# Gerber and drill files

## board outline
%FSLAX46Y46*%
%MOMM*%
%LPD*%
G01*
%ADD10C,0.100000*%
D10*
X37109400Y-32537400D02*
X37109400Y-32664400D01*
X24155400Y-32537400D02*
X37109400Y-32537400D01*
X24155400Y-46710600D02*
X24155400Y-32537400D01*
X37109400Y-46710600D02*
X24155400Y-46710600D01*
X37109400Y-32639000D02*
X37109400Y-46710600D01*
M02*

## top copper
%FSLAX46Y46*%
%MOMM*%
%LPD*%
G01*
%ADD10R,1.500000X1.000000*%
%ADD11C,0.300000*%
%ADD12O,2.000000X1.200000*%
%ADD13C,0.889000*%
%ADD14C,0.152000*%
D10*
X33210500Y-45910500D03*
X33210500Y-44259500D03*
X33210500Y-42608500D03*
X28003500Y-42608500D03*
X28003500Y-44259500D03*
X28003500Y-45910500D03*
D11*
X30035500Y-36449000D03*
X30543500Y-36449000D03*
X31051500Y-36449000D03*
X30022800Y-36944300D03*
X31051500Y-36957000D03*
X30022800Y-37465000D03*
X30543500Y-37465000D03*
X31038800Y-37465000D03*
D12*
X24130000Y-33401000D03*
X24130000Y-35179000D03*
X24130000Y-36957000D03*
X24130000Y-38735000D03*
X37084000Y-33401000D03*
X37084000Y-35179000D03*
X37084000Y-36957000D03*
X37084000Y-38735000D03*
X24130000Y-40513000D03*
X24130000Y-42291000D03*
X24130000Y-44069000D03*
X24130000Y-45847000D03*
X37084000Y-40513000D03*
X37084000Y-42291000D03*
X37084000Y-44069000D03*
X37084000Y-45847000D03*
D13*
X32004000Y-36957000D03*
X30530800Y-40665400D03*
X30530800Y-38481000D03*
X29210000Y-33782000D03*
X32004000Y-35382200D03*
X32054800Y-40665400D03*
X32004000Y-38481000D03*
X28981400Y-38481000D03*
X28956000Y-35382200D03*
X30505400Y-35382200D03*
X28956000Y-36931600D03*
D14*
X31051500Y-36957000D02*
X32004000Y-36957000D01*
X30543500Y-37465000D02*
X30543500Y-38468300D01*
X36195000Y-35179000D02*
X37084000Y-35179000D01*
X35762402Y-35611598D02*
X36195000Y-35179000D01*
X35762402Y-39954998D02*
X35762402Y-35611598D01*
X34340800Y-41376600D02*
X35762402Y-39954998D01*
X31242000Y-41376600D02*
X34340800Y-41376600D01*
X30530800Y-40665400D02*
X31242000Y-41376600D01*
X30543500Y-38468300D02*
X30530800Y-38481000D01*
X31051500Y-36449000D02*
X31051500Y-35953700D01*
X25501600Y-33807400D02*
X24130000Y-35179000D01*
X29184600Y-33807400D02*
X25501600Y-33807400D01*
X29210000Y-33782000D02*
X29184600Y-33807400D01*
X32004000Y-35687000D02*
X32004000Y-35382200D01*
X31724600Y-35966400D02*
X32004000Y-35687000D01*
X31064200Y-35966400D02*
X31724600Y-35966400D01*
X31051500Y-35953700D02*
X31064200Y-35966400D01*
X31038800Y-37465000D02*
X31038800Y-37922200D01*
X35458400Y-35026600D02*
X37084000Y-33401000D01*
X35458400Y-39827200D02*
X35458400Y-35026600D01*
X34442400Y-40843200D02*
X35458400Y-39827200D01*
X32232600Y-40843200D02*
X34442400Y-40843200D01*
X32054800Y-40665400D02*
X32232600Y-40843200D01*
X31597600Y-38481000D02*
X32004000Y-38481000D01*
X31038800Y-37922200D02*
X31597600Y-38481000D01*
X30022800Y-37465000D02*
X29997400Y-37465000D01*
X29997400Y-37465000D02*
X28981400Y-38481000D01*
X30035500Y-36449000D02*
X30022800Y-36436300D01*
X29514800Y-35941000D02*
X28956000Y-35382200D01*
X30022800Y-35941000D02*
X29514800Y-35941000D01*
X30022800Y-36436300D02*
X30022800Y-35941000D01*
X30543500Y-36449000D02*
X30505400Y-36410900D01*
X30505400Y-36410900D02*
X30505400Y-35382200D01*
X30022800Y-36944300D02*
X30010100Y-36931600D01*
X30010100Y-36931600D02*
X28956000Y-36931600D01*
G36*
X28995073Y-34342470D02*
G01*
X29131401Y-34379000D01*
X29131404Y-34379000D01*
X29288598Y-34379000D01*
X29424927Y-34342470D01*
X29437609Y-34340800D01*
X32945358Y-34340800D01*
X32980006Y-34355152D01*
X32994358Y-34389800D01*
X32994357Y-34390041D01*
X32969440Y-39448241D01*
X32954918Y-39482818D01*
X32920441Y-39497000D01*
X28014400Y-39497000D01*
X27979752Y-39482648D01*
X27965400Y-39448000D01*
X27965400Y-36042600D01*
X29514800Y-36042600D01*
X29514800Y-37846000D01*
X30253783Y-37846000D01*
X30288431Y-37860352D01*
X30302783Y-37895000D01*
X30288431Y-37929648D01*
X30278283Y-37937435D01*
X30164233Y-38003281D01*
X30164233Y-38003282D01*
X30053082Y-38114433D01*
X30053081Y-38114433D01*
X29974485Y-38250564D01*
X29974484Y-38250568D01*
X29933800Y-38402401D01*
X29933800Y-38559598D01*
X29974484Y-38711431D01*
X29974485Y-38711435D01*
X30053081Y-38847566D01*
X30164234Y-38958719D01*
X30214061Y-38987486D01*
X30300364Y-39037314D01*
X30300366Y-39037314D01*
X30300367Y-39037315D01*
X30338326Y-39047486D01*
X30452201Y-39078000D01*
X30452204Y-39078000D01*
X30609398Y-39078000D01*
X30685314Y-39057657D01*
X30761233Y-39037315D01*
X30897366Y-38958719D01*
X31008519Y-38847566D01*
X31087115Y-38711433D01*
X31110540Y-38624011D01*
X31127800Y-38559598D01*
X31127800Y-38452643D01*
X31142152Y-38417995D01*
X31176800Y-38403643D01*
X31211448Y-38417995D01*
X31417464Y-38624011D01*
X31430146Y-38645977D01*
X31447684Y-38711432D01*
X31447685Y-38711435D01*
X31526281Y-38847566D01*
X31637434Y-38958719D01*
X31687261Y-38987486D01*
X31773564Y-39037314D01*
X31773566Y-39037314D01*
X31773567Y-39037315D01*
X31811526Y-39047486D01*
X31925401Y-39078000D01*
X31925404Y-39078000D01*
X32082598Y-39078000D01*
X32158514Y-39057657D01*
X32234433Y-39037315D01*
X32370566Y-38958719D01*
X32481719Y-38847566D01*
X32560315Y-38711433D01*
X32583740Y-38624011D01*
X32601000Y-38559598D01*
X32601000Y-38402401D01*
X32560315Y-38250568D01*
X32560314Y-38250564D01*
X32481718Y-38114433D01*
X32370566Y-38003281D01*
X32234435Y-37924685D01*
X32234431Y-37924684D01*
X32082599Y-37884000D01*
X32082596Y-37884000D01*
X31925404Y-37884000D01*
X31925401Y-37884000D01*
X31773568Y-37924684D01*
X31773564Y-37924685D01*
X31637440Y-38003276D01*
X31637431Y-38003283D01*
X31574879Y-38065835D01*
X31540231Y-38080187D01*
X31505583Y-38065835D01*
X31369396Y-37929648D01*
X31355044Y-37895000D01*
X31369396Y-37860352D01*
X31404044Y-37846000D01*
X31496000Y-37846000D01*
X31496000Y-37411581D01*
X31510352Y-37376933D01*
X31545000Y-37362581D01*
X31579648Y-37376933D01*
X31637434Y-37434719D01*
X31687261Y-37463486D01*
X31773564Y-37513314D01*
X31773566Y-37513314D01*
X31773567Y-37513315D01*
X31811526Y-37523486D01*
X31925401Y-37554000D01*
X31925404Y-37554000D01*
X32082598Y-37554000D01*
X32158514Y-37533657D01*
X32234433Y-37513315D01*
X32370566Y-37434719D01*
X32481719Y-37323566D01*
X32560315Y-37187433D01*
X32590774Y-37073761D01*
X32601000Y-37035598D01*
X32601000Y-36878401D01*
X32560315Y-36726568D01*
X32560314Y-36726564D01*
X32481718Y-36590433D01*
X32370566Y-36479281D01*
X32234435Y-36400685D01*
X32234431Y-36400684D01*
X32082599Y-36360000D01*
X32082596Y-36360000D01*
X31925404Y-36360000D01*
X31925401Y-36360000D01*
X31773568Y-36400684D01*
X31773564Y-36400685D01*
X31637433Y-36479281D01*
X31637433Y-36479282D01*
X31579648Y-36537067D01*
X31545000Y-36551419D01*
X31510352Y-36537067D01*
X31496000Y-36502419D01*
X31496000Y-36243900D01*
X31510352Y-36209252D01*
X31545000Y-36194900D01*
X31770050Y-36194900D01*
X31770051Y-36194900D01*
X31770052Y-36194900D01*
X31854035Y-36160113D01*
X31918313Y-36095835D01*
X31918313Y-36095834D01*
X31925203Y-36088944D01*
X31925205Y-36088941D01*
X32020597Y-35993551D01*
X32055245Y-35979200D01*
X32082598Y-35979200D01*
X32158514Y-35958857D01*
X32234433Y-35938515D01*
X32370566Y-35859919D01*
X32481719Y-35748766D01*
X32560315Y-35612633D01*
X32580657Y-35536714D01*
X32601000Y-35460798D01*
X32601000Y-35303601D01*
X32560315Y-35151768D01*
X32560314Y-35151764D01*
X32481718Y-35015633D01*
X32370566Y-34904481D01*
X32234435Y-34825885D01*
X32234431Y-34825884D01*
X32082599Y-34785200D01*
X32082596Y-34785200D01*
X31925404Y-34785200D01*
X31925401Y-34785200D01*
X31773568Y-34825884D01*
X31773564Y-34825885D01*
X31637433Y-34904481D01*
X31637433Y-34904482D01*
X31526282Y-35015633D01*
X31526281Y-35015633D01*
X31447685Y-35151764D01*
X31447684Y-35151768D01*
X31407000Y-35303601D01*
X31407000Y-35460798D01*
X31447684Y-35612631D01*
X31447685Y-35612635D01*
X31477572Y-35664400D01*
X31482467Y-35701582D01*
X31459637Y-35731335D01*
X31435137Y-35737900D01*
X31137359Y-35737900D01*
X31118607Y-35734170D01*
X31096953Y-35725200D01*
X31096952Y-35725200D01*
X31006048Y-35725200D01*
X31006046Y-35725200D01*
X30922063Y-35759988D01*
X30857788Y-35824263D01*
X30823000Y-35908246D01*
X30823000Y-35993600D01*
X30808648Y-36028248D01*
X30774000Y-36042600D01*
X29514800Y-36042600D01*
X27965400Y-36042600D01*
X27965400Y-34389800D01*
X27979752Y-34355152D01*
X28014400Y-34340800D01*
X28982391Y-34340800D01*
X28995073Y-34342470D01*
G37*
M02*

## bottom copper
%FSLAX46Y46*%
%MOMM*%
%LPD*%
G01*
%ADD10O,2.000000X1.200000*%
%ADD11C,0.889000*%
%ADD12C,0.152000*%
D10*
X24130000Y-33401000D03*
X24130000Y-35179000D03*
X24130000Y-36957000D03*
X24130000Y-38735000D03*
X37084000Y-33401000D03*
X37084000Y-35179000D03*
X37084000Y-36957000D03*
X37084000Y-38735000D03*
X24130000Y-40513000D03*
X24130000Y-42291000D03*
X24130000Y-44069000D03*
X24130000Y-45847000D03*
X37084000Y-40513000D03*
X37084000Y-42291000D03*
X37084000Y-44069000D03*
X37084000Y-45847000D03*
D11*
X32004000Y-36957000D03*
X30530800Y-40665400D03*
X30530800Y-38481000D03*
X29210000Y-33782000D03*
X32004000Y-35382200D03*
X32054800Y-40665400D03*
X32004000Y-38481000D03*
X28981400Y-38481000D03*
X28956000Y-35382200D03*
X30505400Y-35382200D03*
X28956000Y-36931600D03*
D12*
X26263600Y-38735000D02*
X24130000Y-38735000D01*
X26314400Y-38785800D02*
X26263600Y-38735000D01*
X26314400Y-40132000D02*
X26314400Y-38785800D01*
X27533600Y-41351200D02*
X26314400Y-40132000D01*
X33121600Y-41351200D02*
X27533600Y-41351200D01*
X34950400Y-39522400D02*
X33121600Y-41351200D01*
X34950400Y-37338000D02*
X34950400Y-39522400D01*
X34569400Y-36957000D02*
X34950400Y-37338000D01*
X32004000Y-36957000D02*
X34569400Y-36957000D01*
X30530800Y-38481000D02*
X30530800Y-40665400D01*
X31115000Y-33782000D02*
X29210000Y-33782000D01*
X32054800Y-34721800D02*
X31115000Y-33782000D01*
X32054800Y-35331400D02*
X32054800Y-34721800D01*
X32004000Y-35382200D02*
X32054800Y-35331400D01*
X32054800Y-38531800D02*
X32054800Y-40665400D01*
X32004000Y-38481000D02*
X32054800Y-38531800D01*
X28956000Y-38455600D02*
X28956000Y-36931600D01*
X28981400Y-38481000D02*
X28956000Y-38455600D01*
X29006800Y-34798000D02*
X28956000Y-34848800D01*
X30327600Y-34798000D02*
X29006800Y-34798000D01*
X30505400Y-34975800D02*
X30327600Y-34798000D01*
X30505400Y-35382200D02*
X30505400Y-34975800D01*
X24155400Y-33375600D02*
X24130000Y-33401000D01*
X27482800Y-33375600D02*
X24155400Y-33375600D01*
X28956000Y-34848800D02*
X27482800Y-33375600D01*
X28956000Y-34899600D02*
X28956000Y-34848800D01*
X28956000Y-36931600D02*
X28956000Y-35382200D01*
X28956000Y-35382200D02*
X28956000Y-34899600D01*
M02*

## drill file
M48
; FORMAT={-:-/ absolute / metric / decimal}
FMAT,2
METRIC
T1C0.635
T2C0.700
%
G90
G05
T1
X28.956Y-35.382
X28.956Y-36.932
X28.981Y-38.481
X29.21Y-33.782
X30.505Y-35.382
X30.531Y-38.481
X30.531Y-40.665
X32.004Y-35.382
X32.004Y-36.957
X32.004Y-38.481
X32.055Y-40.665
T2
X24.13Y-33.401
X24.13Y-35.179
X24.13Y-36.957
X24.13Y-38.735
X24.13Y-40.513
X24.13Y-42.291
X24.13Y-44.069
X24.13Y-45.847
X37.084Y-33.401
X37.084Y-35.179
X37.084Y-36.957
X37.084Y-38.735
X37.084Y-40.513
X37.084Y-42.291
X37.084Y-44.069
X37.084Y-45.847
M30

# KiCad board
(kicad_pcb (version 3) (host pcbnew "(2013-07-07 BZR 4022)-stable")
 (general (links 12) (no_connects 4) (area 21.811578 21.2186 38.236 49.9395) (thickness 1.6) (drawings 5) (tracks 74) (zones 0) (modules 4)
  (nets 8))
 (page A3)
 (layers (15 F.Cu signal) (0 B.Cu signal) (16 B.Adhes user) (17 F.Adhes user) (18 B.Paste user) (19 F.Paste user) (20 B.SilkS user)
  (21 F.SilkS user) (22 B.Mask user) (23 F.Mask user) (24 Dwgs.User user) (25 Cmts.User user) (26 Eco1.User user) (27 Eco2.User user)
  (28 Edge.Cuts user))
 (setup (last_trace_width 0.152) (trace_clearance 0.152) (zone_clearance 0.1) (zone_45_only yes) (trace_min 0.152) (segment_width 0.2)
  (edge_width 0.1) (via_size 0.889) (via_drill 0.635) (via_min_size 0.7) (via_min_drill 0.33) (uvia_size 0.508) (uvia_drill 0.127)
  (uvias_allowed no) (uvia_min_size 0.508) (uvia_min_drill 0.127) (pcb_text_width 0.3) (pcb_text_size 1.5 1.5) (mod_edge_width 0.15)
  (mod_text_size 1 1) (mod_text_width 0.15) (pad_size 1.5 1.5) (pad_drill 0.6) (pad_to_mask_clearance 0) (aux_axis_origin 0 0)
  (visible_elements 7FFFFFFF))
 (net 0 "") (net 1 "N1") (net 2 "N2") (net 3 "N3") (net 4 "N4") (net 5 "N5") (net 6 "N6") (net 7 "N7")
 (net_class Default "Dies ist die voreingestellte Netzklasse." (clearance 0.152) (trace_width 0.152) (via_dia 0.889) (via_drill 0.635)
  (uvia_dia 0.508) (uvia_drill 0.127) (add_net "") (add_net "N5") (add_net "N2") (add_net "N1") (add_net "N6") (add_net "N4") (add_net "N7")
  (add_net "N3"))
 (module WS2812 (layer F.Cu) (at 30.6705 44.2595)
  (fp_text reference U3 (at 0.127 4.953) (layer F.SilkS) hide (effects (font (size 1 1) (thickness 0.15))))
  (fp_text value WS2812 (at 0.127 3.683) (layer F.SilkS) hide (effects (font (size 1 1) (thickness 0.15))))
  (pad 1 smd rect (at 2.54 1.651) (size 1.5 1) (layers F.Cu F.Paste F.Mask))
  (pad 2 smd rect (at 2.54 0) (size 1.5 1) (layers F.Cu F.Paste F.Mask) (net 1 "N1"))
  (pad 3 smd rect (at 2.54 -1.651) (size 1.5 1) (layers F.Cu F.Paste F.Mask) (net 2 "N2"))
  (pad 4 smd rect (at -2.667 -1.651) (size 1.5 1) (layers F.Cu F.Paste F.Mask))
  (pad 5 smd rect (at -2.667 0) (size 1.5 1) (layers F.Cu F.Paste F.Mask) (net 2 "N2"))
  (pad 6 smd rect (at -2.667 1.651) (size 1.5 1) (layers F.Cu F.Paste F.Mask) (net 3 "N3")))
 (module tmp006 (layer F.Cu) (at 30.5435 36.449)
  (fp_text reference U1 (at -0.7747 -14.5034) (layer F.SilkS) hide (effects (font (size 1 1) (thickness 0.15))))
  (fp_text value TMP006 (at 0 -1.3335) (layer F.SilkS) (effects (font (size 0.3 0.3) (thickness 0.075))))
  (pad 1 smd circle (at -0.508 0) (size 0.3 0.3) (layers F.Cu F.Paste F.Mask) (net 3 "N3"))
  (pad 2 smd circle (at 0 0) (size 0.3 0.3) (layers F.Cu F.Paste F.Mask) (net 3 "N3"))
  (pad 3 smd circle (at 0.508 0) (size 0.3 0.3) (layers F.Cu F.Paste F.Mask) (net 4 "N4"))
  (pad 4 smd circle (at -0.5207 0.4953) (size 0.3 0.3) (layers F.Cu F.Paste F.Mask) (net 3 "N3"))
  (pad 5 smd circle (at 0.508 0.508) (size 0.3 0.3) (layers F.Cu F.Paste F.Mask) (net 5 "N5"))
  (pad 6 smd circle (at -0.5207 1.016) (size 0.3 0.3) (layers F.Cu F.Paste F.Mask) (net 3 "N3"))
  (pad 7 smd circle (at 0 1.016) (size 0.3 0.3) (layers F.Cu F.Paste F.Mask) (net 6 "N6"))
  (pad 8 smd circle (at 0.4953 1.016) (size 0.3 0.3) (layers F.Cu F.Paste F.Mask) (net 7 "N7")))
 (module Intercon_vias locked (layer F.Cu) (at 30.607 40.132)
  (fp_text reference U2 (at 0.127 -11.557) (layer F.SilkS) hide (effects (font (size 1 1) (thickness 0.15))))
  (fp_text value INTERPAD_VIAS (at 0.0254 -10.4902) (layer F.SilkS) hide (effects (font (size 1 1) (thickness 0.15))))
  (pad 1 thru_hole oval (at -6.477 -6.731) (size 2 1.2) (drill 0.7) (layers *.Cu *.Mask F.SilkS) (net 3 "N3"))
  (pad 2 thru_hole oval (at -6.477 -4.953) (size 2 1.2) (drill 0.7) (layers *.Cu *.Mask F.SilkS) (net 4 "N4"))
  (pad 3 thru_hole oval (at -6.477 -3.175) (size 2 1.2) (drill 0.7) (layers *.Cu *.Mask F.SilkS))
  (pad 4 thru_hole oval (at -6.477 -1.397) (size 2 1.2) (drill 0.7) (layers *.Cu *.Mask F.SilkS) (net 5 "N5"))
  (pad 5 thru_hole oval (at 6.477 -6.731) (size 2 1.2) (drill 0.7) (layers *.Cu *.Mask F.SilkS) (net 7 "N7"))
  (pad 6 thru_hole oval (at 6.477 -4.953) (size 2 1.2) (drill 0.7) (layers *.Cu *.Mask F.SilkS) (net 6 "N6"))
  (pad 7 thru_hole oval (at 6.477 -3.175) (size 2 1.2) (drill 0.7) (layers *.Cu *.Mask F.SilkS) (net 2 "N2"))
  (pad 8 thru_hole oval (at 6.477 -1.397) (size 2 1.2) (drill 0.7) (layers *.Cu *.Mask F.SilkS) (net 1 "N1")))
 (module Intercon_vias (layer F.Cu) (at 30.607 47.244)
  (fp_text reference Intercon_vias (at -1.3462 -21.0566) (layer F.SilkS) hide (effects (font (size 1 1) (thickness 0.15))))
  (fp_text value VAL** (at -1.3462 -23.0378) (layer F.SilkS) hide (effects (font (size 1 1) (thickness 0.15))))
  (pad 1 thru_hole oval (at -6.477 -6.731) (size 2 1.2) (drill 0.7) (layers *.Cu *.Mask F.SilkS))
  (pad 2 thru_hole oval (at -6.477 -4.953) (size 2 1.2) (drill 0.7) (layers *.Cu *.Mask F.SilkS))
  (pad 3 thru_hole oval (at -6.477 -3.175) (size 2 1.2) (drill 0.7) (layers *.Cu *.Mask F.SilkS))
  (pad 4 thru_hole oval (at -6.477 -1.397) (size 2 1.2) (drill 0.7) (layers *.Cu *.Mask F.SilkS))
  (pad 5 thru_hole oval (at 6.477 -6.731) (size 2 1.2) (drill 0.7) (layers *.Cu *.Mask F.SilkS))
  (pad 6 thru_hole oval (at 6.477 -4.953) (size 2 1.2) (drill 0.7) (layers *.Cu *.Mask F.SilkS))
  (pad 7 thru_hole oval (at 6.477 -3.175) (size 2 1.2) (drill 0.7) (layers *.Cu *.Mask F.SilkS))
  (pad 8 thru_hole oval (at 6.477 -1.397) (size 2 1.2) (drill 0.7) (layers *.Cu *.Mask F.SilkS)))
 (gr_line (start 37.1094 32.5374) (end 37.1094 32.6644) (angle 90) (layer Edge.Cuts) (width 0.1))
 (gr_line (start 24.1554 32.5374) (end 37.1094 32.5374) (angle 90) (layer Edge.Cuts) (width 0.1))
 (gr_line (start 24.1554 46.7106) (end 24.1554 32.5374) (angle 90) (layer Edge.Cuts) (width 0.1))
 (gr_line (start 37.1094 46.7106) (end 24.1554 46.7106) (angle 90) (layer Edge.Cuts) (width 0.1))
 (gr_line (start 37.1094 32.639) (end 37.1094 46.7106) (angle 90) (layer Edge.Cuts) (width 0.1))
 (segment (start 31.0515 36.957) (end 32.004 36.957) (width 0.152) (layer F.Cu) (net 5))
 (segment (start 26.2636 38.735) (end 24.13 38.735) (width 0.152) (layer B.Cu) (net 5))
 (segment (start 26.3144 38.7858) (end 26.2636 38.735) (width 0.152) (layer B.Cu) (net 5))
 (segment (start 26.3144 40.132) (end 26.3144 38.7858) (width 0.152) (layer B.Cu) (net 5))
 (segment (start 27.5336 41.3512) (end 26.3144 40.132) (width 0.152) (layer B.Cu) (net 5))
 (segment (start 33.1216 41.3512) (end 27.5336 41.3512) (width 0.152) (layer B.Cu) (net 5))
 (segment (start 34.9504 39.5224) (end 33.1216 41.3512) (width 0.152) (layer B.Cu) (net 5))
 (segment (start 34.9504 37.338) (end 34.9504 39.5224) (width 0.152) (layer B.Cu) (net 5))
 (segment (start 34.5694 36.957) (end 34.9504 37.338) (width 0.152) (layer B.Cu) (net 5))
 (segment (start 32.004 36.957) (end 34.5694 36.957) (width 0.152) (layer B.Cu) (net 5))
 (via (at 32.004 36.957) (size 0.889) (layers F.Cu B.Cu) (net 5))
 (segment (start 30.5435 37.465) (end 30.5435 38.4683) (width 0.152) (layer F.Cu) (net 6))
 (segment (start 36.195 35.179) (end 37.084 35.179) (width 0.152) (layer F.Cu) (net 6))
 (segment (start 35.762402 35.611598) (end 36.195 35.179) (width 0.152) (layer F.Cu) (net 6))
 (segment (start 35.762402 39.954998) (end 35.762402 35.611598) (width 0.152) (layer F.Cu) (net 6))
 (segment (start 34.3408 41.3766) (end 35.762402 39.954998) (width 0.152) (layer F.Cu) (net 6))
 (segment (start 31.242 41.3766) (end 34.3408 41.3766) (width 0.152) (layer F.Cu) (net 6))
 (segment (start 30.5308 40.6654) (end 31.242 41.3766) (width 0.152) (layer F.Cu) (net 6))
 (via (at 30.5308 40.6654) (size 0.889) (layers F.Cu B.Cu) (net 6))
 (segment (start 30.5308 38.481) (end 30.5308 40.6654) (width 0.152) (layer B.Cu) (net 6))
 (via (at 30.5308 38.481) (size 0.889) (layers F.Cu B.Cu) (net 6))
 (segment (start 30.5435 38.4683) (end 30.5308 38.481) (width 0.152) (layer F.Cu) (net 6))
 (segment (start 31.0515 36.449) (end 31.0515 35.9537) (width 0.152) (layer F.Cu) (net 4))
 (segment (start 25.5016 33.8074) (end 24.13 35.179) (width 0.152) (layer F.Cu) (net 4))
 (segment (start 29.1846 33.8074) (end 25.5016 33.8074) (width 0.152) (layer F.Cu) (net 4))
 (segment (start 29.21 33.782) (end 29.1846 33.8074) (width 0.152) (layer F.Cu) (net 4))
 (via (at 29.21 33.782) (size 0.889) (layers F.Cu B.Cu) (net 4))
 (segment (start 31.115 33.782) (end 29.21 33.782) (width 0.152) (layer B.Cu) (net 4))
 (segment (start 32.0548 34.7218) (end 31.115 33.782) (width 0.152) (layer B.Cu) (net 4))
 (segment (start 32.0548 35.3314) (end 32.0548 34.7218) (width 0.152) (layer B.Cu) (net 4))
 (segment (start 32.004 35.3822) (end 32.0548 35.3314) (width 0.152) (layer B.Cu) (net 4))
 (via (at 32.004 35.3822) (size 0.889) (layers F.Cu B.Cu) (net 4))
 (segment (start 32.004 35.687) (end 32.004 35.3822) (width 0.152) (layer F.Cu) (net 4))
 (segment (start 31.7246 35.9664) (end 32.004 35.687) (width 0.152) (layer F.Cu) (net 4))
 (segment (start 31.0642 35.9664) (end 31.7246 35.9664) (width 0.152) (layer F.Cu) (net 4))
 (segment (start 31.0515 35.9537) (end 31.0642 35.9664) (width 0.152) (layer F.Cu) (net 4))
 (segment (start 31.0388 37.465) (end 31.0388 37.9222) (width 0.152) (layer F.Cu) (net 7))
 (segment (start 35.4584 35.0266) (end 37.084 33.401) (width 0.152) (layer F.Cu) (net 7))
 (segment (start 35.4584 39.8272) (end 35.4584 35.0266) (width 0.152) (layer F.Cu) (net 7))
 (segment (start 34.4424 40.8432) (end 35.4584 39.8272) (width 0.152) (layer F.Cu) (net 7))
 (segment (start 32.2326 40.8432) (end 34.4424 40.8432) (width 0.152) (layer F.Cu) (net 7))
 (segment (start 32.0548 40.6654) (end 32.2326 40.8432) (width 0.152) (layer F.Cu) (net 7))
 (via (at 32.0548 40.6654) (size 0.889) (layers F.Cu B.Cu) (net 7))
 (segment (start 32.0548 38.5318) (end 32.0548 40.6654) (width 0.152) (layer B.Cu) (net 7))
 (segment (start 32.004 38.481) (end 32.0548 38.5318) (width 0.152) (layer B.Cu) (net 7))
 (via (at 32.004 38.481) (size 0.889) (layers F.Cu B.Cu) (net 7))
 (segment (start 31.5976 38.481) (end 32.004 38.481) (width 0.152) (layer F.Cu) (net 7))
 (segment (start 31.0388 37.9222) (end 31.5976 38.481) (width 0.152) (layer F.Cu) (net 7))
 (segment (start 30.0228 37.465) (end 29.9974 37.465) (width 0.152) (layer F.Cu) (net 3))
 (segment (start 28.956 38.4556) (end 28.956 36.9316) (width 0.152) (layer B.Cu) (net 3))
 (segment (start 28.9814 38.481) (end 28.956 38.4556) (width 0.152) (layer B.Cu) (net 3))
 (via (at 28.9814 38.481) (size 0.889) (layers F.Cu B.Cu) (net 3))
 (segment (start 29.9974 37.465) (end 28.9814 38.481) (width 0.152) (layer F.Cu) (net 3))
 (segment (start 30.0355 36.449) (end 30.0228 36.4363) (width 0.152) (layer F.Cu) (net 3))
 (via (at 28.956 35.3822) (size 0.889) (layers F.Cu B.Cu) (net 3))
 (segment (start 29.5148 35.941) (end 28.956 35.3822) (width 0.152) (layer F.Cu) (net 3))
 (segment (start 30.0228 35.941) (end 29.5148 35.941) (width 0.152) (layer F.Cu) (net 3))
 (segment (start 30.0228 36.4363) (end 30.0228 35.941) (width 0.152) (layer F.Cu) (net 3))
 (segment (start 30.5435 36.449) (end 30.5054 36.4109) (width 0.152) (layer F.Cu) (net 3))
 (segment (start 29.0068 34.798) (end 28.956 34.8488) (width 0.152) (layer B.Cu) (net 3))
 (segment (start 30.3276 34.798) (end 29.0068 34.798) (width 0.152) (layer B.Cu) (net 3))
 (segment (start 30.5054 34.9758) (end 30.3276 34.798) (width 0.152) (layer B.Cu) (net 3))
 (segment (start 30.5054 35.3822) (end 30.5054 34.9758) (width 0.152) (layer B.Cu) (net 3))
 (via (at 30.5054 35.3822) (size 0.889) (layers F.Cu B.Cu) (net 3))
 (segment (start 30.5054 36.4109) (end 30.5054 35.3822) (width 0.152) (layer F.Cu) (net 3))
 (segment (start 30.0228 36.9443) (end 30.0101 36.9316) (width 0.152) (layer F.Cu) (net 3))
 (segment (start 30.0101 36.9316) (end 28.956 36.9316) (width 0.152) (layer F.Cu) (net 3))
 (segment (start 24.1554 33.3756) (end 24.13 33.401) (width 0.152) (layer B.Cu) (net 3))
 (segment (start 27.4828 33.3756) (end 24.1554 33.3756) (width 0.152) (layer B.Cu) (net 3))
 (segment (start 28.956 34.8488) (end 27.4828 33.3756) (width 0.152) (layer B.Cu) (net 3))
 (segment (start 28.956 34.8996) (end 28.956 34.8488) (width 0.152) (layer B.Cu) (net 3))
 (segment (start 28.956 36.9316) (end 28.956 35.3822) (width 0.152) (layer B.Cu) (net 3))
 (segment (start 28.956 35.3822) (end 28.956 34.8996) (width 0.152) (layer B.Cu) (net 3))
 (via (at 28.956 36.9316) (size 0.889) (layers F.Cu B.Cu) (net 3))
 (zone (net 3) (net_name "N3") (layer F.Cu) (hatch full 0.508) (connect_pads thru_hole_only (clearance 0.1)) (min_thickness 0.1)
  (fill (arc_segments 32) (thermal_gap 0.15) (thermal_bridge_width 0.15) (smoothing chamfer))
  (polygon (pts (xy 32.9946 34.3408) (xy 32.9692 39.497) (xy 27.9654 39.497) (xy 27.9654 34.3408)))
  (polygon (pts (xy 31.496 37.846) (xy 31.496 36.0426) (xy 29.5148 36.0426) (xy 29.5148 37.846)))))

